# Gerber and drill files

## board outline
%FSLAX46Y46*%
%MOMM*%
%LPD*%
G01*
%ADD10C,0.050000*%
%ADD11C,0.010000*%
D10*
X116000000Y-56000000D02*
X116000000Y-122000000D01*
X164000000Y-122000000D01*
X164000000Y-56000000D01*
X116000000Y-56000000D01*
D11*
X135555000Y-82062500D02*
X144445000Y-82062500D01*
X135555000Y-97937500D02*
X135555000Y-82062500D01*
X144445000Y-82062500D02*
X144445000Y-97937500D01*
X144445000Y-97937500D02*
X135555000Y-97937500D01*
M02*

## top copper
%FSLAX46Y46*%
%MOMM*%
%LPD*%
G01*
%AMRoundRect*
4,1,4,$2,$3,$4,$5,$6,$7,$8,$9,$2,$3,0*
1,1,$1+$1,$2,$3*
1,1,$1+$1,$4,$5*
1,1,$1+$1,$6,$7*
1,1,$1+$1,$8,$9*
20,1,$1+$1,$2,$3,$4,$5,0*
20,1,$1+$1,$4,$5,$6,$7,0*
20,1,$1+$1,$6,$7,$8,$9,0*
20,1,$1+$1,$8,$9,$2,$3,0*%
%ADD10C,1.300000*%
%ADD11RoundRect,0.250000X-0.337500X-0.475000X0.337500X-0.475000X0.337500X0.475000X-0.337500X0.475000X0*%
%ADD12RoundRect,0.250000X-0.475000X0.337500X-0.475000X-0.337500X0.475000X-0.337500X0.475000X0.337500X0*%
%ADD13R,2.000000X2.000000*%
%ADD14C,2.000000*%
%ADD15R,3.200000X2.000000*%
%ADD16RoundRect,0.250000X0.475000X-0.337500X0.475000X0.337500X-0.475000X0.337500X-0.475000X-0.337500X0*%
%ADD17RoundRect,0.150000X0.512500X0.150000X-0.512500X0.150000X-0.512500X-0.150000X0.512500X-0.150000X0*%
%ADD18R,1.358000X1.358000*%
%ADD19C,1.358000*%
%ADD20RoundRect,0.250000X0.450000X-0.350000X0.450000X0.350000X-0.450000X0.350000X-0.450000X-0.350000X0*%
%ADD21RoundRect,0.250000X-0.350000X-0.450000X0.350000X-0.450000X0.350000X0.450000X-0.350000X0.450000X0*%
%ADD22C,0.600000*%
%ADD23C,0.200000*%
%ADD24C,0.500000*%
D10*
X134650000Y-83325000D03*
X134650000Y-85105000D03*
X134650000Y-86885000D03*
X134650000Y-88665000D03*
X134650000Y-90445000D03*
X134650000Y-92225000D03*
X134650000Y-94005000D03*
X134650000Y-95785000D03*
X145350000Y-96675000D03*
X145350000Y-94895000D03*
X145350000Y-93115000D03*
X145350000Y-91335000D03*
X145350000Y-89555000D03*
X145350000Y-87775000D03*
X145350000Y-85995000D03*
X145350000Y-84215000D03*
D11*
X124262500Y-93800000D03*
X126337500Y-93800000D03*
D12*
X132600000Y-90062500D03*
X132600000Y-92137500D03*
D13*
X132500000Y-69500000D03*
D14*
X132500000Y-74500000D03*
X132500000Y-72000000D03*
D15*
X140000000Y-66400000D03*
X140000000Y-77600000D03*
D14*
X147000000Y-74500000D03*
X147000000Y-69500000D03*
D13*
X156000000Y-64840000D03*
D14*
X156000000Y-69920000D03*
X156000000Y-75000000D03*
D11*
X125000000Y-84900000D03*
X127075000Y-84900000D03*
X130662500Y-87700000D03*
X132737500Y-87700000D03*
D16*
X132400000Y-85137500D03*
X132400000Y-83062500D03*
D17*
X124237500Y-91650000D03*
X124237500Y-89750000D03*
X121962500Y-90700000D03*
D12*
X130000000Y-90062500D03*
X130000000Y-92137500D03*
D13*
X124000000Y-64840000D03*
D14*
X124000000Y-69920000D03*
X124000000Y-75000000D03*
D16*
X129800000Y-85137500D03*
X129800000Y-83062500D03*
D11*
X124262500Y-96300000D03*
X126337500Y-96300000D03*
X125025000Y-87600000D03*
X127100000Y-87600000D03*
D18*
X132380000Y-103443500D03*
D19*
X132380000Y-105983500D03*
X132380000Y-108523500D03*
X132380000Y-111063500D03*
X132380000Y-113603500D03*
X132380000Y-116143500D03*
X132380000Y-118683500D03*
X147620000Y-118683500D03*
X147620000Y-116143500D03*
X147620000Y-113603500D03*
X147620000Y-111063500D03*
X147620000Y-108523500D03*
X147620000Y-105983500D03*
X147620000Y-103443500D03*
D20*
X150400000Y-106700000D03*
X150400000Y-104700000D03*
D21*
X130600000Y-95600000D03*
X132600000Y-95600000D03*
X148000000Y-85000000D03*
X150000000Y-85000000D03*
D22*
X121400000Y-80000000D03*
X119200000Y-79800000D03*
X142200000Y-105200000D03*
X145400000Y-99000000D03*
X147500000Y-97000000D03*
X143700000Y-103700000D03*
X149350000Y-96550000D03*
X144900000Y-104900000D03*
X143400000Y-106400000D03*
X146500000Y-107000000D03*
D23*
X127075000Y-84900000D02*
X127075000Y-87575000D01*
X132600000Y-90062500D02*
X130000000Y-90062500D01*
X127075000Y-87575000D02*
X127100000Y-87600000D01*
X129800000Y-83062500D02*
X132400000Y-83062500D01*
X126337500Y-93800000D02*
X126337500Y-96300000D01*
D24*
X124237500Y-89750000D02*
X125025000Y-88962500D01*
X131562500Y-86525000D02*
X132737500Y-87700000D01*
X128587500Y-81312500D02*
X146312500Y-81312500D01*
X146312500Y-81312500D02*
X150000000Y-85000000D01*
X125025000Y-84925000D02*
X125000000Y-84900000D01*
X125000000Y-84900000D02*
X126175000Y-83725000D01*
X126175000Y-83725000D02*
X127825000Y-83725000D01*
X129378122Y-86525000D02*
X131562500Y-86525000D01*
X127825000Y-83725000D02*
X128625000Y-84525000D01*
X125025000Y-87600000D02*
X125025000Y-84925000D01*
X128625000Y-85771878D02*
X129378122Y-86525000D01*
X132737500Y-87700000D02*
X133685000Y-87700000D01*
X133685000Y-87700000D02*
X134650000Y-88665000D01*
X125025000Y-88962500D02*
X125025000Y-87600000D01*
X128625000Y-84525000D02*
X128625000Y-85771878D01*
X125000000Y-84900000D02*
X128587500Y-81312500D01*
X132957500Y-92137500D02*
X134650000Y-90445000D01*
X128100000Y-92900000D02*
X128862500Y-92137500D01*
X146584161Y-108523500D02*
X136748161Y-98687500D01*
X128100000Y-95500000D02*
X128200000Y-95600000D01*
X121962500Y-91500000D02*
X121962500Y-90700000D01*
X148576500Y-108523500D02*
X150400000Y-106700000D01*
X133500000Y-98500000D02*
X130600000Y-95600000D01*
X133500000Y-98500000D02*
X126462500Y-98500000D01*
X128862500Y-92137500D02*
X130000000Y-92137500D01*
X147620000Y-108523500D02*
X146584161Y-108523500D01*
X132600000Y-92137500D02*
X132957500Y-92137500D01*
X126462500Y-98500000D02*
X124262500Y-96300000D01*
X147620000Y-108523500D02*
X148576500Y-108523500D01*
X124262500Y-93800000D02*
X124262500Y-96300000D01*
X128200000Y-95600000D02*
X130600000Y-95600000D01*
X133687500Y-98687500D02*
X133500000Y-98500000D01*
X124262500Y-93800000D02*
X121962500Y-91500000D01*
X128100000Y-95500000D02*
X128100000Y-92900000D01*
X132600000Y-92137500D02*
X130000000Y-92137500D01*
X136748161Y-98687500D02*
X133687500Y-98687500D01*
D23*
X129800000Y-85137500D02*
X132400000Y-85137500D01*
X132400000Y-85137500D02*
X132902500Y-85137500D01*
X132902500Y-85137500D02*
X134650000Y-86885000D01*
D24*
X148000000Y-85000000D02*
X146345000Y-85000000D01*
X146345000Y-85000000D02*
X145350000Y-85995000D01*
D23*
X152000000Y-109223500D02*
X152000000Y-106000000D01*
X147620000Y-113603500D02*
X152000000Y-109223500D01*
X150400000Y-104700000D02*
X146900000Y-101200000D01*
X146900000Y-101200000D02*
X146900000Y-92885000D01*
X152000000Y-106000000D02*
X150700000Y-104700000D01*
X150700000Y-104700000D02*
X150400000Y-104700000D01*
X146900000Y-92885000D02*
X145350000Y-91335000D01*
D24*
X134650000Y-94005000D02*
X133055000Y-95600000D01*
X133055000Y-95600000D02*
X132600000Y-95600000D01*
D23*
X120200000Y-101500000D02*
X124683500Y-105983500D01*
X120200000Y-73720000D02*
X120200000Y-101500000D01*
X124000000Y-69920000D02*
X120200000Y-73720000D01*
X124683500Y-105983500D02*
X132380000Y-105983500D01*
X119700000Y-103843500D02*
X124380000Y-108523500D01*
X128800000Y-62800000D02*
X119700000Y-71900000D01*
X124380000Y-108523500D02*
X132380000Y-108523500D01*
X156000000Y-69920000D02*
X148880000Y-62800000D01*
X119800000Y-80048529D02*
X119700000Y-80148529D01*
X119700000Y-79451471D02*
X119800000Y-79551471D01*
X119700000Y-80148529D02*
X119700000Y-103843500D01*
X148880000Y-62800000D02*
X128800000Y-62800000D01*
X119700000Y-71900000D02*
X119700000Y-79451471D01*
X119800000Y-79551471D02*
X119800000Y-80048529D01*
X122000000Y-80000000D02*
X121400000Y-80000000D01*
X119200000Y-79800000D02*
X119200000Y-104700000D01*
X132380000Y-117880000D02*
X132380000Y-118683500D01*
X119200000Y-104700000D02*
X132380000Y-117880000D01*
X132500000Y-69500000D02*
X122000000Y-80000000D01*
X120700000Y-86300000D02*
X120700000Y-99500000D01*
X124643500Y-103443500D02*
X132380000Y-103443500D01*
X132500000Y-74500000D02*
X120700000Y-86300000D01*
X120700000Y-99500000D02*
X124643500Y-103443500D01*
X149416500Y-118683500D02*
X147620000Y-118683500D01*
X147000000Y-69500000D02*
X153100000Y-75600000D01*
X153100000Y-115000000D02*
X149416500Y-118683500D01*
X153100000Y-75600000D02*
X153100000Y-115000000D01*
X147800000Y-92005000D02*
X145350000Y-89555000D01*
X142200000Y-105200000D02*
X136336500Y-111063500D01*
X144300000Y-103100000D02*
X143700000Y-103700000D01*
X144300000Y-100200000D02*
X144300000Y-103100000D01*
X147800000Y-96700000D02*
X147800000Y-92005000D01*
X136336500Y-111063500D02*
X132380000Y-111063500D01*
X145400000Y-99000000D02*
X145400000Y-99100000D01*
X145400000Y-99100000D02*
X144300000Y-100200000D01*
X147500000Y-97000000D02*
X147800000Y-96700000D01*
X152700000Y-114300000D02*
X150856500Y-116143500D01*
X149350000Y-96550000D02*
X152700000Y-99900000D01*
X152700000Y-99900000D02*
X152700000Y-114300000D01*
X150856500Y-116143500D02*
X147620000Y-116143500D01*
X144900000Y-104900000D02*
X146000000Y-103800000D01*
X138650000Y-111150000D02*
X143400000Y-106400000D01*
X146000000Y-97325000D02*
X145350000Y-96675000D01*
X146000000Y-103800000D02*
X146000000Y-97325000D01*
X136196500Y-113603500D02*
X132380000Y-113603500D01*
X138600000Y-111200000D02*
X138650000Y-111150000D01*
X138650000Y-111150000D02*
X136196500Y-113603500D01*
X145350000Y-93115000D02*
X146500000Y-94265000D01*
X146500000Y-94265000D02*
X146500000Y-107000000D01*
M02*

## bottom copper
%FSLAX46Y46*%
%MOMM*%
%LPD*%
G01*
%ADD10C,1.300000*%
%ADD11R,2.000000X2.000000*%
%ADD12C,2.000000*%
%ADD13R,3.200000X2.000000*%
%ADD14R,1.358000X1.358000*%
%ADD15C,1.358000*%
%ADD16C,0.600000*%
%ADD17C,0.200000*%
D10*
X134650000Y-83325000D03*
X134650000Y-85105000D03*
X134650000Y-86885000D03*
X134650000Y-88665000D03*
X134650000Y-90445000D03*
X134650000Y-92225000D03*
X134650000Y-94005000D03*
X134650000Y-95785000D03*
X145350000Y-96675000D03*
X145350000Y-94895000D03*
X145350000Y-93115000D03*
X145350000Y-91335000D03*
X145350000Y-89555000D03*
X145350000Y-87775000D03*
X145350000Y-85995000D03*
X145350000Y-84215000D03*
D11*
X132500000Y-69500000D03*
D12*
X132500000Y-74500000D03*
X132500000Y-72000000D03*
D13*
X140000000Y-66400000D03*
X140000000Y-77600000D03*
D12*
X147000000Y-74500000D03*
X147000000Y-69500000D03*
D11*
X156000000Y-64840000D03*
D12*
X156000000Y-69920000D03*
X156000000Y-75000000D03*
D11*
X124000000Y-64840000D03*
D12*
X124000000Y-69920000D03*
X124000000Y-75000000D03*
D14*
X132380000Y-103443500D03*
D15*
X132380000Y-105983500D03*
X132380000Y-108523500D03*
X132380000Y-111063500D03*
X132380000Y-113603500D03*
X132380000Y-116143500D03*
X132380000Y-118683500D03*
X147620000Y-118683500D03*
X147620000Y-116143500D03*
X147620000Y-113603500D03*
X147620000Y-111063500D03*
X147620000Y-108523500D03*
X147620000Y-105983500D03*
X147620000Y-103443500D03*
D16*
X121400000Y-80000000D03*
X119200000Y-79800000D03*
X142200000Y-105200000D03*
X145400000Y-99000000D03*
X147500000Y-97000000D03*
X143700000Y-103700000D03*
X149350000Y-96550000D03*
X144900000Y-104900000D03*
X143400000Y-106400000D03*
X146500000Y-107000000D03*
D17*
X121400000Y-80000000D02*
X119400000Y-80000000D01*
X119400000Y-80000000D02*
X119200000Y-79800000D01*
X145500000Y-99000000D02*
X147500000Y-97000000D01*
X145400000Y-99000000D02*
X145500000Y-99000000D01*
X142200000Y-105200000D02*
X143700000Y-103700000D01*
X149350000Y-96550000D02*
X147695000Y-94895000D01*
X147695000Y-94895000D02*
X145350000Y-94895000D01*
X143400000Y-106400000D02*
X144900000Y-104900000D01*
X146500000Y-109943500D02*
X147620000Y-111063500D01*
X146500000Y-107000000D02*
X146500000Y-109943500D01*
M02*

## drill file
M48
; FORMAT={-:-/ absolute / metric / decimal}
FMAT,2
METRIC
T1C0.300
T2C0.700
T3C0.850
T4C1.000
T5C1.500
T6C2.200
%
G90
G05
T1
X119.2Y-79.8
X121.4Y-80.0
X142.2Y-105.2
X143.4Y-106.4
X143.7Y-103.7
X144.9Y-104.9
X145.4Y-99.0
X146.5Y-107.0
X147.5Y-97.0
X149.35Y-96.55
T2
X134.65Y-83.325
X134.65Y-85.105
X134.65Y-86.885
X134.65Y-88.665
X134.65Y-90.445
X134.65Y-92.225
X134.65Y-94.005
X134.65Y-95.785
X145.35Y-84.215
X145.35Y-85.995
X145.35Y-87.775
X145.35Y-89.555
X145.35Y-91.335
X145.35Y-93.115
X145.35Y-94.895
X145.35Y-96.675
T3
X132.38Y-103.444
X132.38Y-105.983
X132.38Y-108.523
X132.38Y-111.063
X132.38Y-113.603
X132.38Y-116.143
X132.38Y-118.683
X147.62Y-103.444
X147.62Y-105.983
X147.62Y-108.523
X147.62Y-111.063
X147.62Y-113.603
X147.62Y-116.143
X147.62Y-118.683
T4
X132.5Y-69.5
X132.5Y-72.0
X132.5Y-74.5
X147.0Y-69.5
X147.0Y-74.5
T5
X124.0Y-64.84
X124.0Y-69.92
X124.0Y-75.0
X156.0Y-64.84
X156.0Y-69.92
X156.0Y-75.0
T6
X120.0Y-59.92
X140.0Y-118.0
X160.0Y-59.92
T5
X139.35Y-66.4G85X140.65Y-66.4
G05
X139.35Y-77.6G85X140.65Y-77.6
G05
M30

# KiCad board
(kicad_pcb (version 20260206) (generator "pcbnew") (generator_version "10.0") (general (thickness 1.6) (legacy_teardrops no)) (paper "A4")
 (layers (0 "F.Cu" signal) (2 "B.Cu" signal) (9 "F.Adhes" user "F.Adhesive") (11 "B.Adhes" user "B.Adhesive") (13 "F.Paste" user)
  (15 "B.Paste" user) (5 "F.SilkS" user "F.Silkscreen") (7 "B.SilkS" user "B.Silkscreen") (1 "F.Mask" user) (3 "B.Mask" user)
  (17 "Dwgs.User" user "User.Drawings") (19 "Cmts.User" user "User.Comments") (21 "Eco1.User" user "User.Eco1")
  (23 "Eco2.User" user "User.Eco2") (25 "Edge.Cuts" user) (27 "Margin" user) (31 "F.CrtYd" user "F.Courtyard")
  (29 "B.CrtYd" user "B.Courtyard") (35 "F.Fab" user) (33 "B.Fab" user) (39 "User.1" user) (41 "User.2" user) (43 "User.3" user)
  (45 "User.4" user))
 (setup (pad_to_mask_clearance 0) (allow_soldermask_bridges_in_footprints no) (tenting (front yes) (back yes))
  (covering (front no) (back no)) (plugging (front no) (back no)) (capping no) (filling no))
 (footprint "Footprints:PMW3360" (layer "F.Cu") (at 140 90)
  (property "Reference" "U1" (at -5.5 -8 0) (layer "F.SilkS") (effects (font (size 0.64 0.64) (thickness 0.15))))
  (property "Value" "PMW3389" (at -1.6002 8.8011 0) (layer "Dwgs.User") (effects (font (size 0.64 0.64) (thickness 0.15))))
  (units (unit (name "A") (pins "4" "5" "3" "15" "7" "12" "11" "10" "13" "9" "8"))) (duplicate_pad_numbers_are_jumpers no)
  (fp_line (start -4.445 -7.9375) (end 4.445 -7.9375) (stroke (width 0.01) (type solid)) (layer "Edge.Cuts"))
  (fp_line (start -4.445 7.9375) (end -4.445 -7.9375) (stroke (width 0.01) (type solid)) (layer "Edge.Cuts"))
  (fp_line (start 4.445 -7.9375) (end 4.445 7.9375) (stroke (width 0.01) (type solid)) (layer "Edge.Cuts"))
  (fp_line (start 4.445 7.9375) (end -4.445 7.9375) (stroke (width 0.01) (type solid)) (layer "Edge.Cuts"))
  (pad "1" thru_hole circle (at -5.35 -6.675) (size 1.3 1.3) (drill 0.7) (layers "*.Cu" "*.Mask") (remove_unused_layers no)
   (solder_mask_margin 0.102))
  (pad "2" thru_hole circle (at -5.35 -4.895) (size 1.3 1.3) (drill 0.7) (layers "*.Cu" "*.Mask") (remove_unused_layers no)
   (solder_mask_margin 0.102))
  (pad "3" thru_hole circle (at -5.35 -3.115) (size 1.3 1.3) (drill 0.7) (layers "*.Cu" "*.Mask") (remove_unused_layers no)
   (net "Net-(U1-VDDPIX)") (solder_mask_margin 0.102))
  (pad "4" thru_hole circle (at -5.35 -1.335) (size 1.3 1.3) (drill 0.7) (layers "*.Cu" "*.Mask") (remove_unused_layers no) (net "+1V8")
   (solder_mask_margin 0.102))
  (pad "5" thru_hole circle (at -5.35 0.445) (size 1.3 1.3) (drill 0.7) (layers "*.Cu" "*.Mask") (remove_unused_layers no) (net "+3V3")
   (solder_mask_margin 0.102))
  (pad "6" thru_hole circle (at -5.35 2.225) (size 1.3 1.3) (drill 0.7) (layers "*.Cu" "*.Mask") (remove_unused_layers no)
   (solder_mask_margin 0.102))
  (pad "7" thru_hole circle (at -5.35 4.005) (size 1.3 1.3) (drill 0.7) (layers "*.Cu" "*.Mask") (remove_unused_layers no)
   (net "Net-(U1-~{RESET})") (solder_mask_margin 0.102))
  (pad "8" thru_hole circle (at -5.35 5.785) (size 1.3 1.3) (drill 0.7) (layers "*.Cu" "*.Mask") (remove_unused_layers no) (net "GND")
   (solder_mask_margin 0.102))
  (pad "9" thru_hole circle (at 5.35 6.675) (size 1.3 1.3) (drill 0.7) (layers "*.Cu" "*.Mask") (remove_unused_layers no) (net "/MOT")
   (solder_mask_margin 0.102))
  (pad "10" thru_hole circle (at 5.35 4.895) (size 1.3 1.3) (drill 0.7) (layers "*.Cu" "*.Mask") (remove_unused_layers no) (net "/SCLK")
   (solder_mask_margin 0.102))
  (pad "11" thru_hole circle (at 5.35 3.115) (size 1.3 1.3) (drill 0.7) (layers "*.Cu" "*.Mask") (remove_unused_layers no) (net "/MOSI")
   (solder_mask_margin 0.102))
  (pad "12" thru_hole circle (at 5.35 1.335) (size 1.3 1.3) (drill 0.7) (layers "*.Cu" "*.Mask") (remove_unused_layers no) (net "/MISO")
   (solder_mask_margin 0.102))
  (pad "13" thru_hole circle (at 5.35 -0.445) (size 1.3 1.3) (drill 0.7) (layers "*.Cu" "*.Mask") (remove_unused_layers no) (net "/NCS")
   (solder_mask_margin 0.102))
  (pad "14" thru_hole circle (at 5.35 -2.225) (size 1.3 1.3) (drill 0.7) (layers "*.Cu" "*.Mask") (remove_unused_layers no)
   (solder_mask_margin 0.102))
  (pad "15" thru_hole circle (at 5.35 -4.005) (size 1.3 1.3) (drill 0.7) (layers "*.Cu" "*.Mask") (remove_unused_layers no)
   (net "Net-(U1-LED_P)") (solder_mask_margin 0.102))
  (pad "16" thru_hole circle (at 5.35 -5.785) (size 1.3 1.3) (drill 0.7) (layers "*.Cu" "*.Mask") (remove_unused_layers no)
   (solder_mask_margin 0.102))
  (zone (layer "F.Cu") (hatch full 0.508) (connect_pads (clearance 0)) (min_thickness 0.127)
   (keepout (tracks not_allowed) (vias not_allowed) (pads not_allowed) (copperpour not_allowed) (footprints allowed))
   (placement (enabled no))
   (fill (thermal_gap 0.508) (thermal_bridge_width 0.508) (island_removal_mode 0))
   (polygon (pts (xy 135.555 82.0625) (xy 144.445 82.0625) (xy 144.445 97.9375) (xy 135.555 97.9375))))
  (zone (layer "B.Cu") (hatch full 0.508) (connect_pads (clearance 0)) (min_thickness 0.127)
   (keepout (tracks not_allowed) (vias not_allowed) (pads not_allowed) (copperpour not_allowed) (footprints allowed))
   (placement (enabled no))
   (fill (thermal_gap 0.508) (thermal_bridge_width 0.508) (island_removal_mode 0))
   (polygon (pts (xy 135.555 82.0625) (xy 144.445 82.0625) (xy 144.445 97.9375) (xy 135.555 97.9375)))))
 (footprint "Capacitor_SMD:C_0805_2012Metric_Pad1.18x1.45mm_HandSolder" (layer "F.Cu") (at 125.3 93.8)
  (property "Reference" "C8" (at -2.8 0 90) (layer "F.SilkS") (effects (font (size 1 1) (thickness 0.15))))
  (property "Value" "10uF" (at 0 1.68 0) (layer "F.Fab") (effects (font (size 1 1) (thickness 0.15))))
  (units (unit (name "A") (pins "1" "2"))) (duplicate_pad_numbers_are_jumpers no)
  (pad "1" smd roundrect (at -1.0375 0) (size 1.175 1.45) (layers "F.Cu" "F.Mask" "F.Paste") (roundrect_rratio 0.212766) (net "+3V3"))
  (pad "2" smd roundrect (at 1.0375 0) (size 1.175 1.45) (layers "F.Cu" "F.Mask" "F.Paste") (roundrect_rratio 0.212766) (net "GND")))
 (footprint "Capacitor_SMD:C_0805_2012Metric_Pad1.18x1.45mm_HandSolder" (layer "F.Cu") (at 132.6 91.1 -90)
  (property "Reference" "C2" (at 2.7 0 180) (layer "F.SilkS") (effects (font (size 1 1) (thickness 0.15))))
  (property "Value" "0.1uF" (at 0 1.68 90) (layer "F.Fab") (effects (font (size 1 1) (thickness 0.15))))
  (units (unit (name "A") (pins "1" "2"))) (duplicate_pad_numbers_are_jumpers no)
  (pad "1" smd roundrect (at -1.0375 0 270) (size 1.175 1.45) (layers "F.Cu" "F.Mask" "F.Paste") (roundrect_rratio 0.212766) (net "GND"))
  (pad "2" smd roundrect (at 1.0375 0 270) (size 1.175 1.45) (layers "F.Cu" "F.Mask" "F.Paste") (roundrect_rratio 0.212766) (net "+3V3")))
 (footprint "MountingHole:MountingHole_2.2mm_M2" (layer "F.Cu") (at 140 118)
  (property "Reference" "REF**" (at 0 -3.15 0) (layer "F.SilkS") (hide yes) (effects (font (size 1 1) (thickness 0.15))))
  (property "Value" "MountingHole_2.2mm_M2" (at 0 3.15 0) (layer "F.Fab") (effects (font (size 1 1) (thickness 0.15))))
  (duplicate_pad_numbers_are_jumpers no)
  (pad "" np_thru_hole circle (at 0 0) (size 2.2 2.2) (drill 2.2) (layers "*.Cu" "*.Mask")))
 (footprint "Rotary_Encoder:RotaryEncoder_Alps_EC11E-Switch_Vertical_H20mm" (layer "F.Cu") (at 132.5 69.5)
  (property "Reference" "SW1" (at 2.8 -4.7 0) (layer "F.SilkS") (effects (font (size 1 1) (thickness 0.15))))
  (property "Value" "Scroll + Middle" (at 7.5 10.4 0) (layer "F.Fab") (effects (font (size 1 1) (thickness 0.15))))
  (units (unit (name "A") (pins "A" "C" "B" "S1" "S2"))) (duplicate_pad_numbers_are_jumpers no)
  (pad "A" thru_hole rect (at 0 0) (size 2 2) (drill 1) (layers "*.Cu" "*.Mask") (remove_unused_layers no) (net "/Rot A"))
  (pad "B" thru_hole circle (at 0 5) (size 2 2) (drill 1) (layers "*.Cu" "*.Mask") (remove_unused_layers no) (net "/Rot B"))
  (pad "C" thru_hole circle (at 0 2.5) (size 2 2) (drill 1) (layers "*.Cu" "*.Mask") (remove_unused_layers no) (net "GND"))
  (pad "MP" thru_hole rect (at 7.5 -3.1) (size 3.2 2) (drill oval 2.8 1.5) (layers "*.Cu" "*.Mask") (remove_unused_layers no))
  (pad "MP" thru_hole rect (at 7.5 8.1) (size 3.2 2) (drill oval 2.8 1.5) (layers "*.Cu" "*.Mask") (remove_unused_layers no))
  (pad "S1" thru_hole circle (at 14.5 5) (size 2 2) (drill 1) (layers "*.Cu" "*.Mask") (remove_unused_layers no) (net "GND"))
  (pad "S2" thru_hole circle (at 14.5 0) (size 2 2) (drill 1) (layers "*.Cu" "*.Mask") (remove_unused_layers no) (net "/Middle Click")))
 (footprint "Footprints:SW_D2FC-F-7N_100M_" (layer "F.Cu") (at 156 69.92 -90)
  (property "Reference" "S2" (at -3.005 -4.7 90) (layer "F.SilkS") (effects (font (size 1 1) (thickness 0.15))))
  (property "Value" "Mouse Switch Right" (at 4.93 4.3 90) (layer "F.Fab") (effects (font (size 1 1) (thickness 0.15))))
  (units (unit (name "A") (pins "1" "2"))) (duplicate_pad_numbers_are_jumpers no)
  (pad "1" thru_hole rect (at -5.08 0 270) (size 2 2) (drill 1.5) (layers "*.Cu" "*.Mask") (remove_unused_layers no) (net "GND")
   (solder_mask_margin 0.102))
  (pad "2" thru_hole circle (at 0 0 270) (size 2 2) (drill 1.5) (layers "*.Cu" "*.Mask") (remove_unused_layers no) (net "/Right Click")
   (solder_mask_margin 0.102))
  (pad "3" thru_hole circle (at 5.08 0 270) (size 2 2) (drill 1.5) (layers "*.Cu" "*.Mask") (remove_unused_layers no)
   (solder_mask_margin 0.102)))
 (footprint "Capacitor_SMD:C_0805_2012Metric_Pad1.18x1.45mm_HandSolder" (layer "F.Cu") (at 126.0375 84.9)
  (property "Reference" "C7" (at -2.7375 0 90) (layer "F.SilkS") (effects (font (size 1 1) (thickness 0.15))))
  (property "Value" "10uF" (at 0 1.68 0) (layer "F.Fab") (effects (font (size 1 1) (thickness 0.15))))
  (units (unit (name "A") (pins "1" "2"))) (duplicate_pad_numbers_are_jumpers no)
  (pad "1" smd roundrect (at -1.0375 0) (size 1.175 1.45) (layers "F.Cu" "F.Mask" "F.Paste") (roundrect_rratio 0.212766) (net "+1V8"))
  (pad "2" smd roundrect (at 1.0375 0) (size 1.175 1.45) (layers "F.Cu" "F.Mask" "F.Paste") (roundrect_rratio 0.212766) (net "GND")))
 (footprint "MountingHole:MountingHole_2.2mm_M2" (layer "F.Cu") (at 120 59.92)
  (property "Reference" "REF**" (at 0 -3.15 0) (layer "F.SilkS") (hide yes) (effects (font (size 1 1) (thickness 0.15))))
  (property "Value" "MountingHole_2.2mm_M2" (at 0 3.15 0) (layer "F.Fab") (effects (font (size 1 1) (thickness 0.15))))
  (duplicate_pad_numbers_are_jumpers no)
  (pad "" np_thru_hole circle (at 0 0) (size 2.2 2.2) (drill 2.2) (layers "*.Cu" "*.Mask")))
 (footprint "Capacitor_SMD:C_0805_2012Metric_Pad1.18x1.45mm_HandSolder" (layer "F.Cu") (at 131.7 87.7)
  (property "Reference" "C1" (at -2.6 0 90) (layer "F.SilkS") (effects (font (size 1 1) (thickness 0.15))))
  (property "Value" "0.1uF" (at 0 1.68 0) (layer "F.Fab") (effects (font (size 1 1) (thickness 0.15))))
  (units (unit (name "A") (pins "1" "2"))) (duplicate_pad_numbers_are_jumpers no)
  (pad "1" smd roundrect (at -1.0375 0) (size 1.175 1.45) (layers "F.Cu" "F.Mask" "F.Paste") (roundrect_rratio 0.212766) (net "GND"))
  (pad "2" smd roundrect (at 1.0375 0) (size 1.175 1.45) (layers "F.Cu" "F.Mask" "F.Paste") (roundrect_rratio 0.212766) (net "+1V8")))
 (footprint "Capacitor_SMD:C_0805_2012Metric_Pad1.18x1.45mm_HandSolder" (layer "F.Cu") (at 132.4 84.1 90)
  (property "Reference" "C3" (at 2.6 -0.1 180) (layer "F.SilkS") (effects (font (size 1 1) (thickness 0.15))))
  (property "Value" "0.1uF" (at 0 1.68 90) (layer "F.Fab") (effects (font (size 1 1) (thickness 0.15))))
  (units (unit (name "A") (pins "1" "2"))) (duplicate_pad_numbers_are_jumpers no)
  (pad "1" smd roundrect (at -1.0375 0 90) (size 1.175 1.45) (layers "F.Cu" "F.Mask" "F.Paste") (roundrect_rratio 0.212766)
   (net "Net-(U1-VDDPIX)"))
  (pad "2" smd roundrect (at 1.0375 0 90) (size 1.175 1.45) (layers "F.Cu" "F.Mask" "F.Paste") (roundrect_rratio 0.212766) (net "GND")))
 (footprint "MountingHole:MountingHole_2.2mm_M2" (layer "F.Cu") (at 160 59.92)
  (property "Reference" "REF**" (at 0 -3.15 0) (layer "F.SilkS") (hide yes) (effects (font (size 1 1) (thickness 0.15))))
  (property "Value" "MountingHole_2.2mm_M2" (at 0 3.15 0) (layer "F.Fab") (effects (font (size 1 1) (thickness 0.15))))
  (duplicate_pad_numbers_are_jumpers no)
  (pad "" np_thru_hole circle (at 0 0) (size 2.2 2.2) (drill 2.2) (layers "*.Cu" "*.Mask")))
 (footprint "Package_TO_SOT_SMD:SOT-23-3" (layer "F.Cu") (at 123.1 90.7 180)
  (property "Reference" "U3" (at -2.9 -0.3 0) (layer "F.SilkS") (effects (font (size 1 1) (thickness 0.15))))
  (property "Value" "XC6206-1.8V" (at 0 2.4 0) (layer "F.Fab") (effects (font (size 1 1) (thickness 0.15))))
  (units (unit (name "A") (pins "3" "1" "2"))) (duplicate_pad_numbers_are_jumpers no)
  (pad "1" smd roundrect (at -1.1375 -0.95 180) (size 1.325 0.6) (layers "F.Cu" "F.Mask" "F.Paste") (roundrect_rratio 0.25) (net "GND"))
  (pad "2" smd roundrect (at -1.1375 0.95 180) (size 1.325 0.6) (layers "F.Cu" "F.Mask" "F.Paste") (roundrect_rratio 0.25) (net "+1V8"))
  (pad "3" smd roundrect (at 1.1375 0 180) (size 1.325 0.6) (layers "F.Cu" "F.Mask" "F.Paste") (roundrect_rratio 0.25) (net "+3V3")))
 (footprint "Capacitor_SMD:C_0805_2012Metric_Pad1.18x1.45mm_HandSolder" (layer "F.Cu") (at 130 91.1 -90)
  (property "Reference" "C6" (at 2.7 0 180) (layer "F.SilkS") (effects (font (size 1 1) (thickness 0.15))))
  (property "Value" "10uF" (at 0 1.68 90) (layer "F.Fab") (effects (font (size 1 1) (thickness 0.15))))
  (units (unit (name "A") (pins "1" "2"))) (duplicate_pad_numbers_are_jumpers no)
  (pad "1" smd roundrect (at -1.0375 0 270) (size 1.175 1.45) (layers "F.Cu" "F.Mask" "F.Paste") (roundrect_rratio 0.212766) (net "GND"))
  (pad "2" smd roundrect (at 1.0375 0 270) (size 1.175 1.45) (layers "F.Cu" "F.Mask" "F.Paste") (roundrect_rratio 0.212766) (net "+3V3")))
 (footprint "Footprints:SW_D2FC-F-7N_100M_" (layer "F.Cu") (at 124 69.92 -90)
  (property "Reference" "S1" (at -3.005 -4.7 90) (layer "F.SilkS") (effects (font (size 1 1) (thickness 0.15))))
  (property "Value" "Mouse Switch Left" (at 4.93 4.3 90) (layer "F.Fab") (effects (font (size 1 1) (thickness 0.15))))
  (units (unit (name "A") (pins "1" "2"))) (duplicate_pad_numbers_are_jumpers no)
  (pad "1" thru_hole rect (at -5.08 0 270) (size 2 2) (drill 1.5) (layers "*.Cu" "*.Mask") (remove_unused_layers no) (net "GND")
   (solder_mask_margin 0.102))
  (pad "2" thru_hole circle (at 0 0 270) (size 2 2) (drill 1.5) (layers "*.Cu" "*.Mask") (remove_unused_layers no) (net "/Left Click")
   (solder_mask_margin 0.102))
  (pad "3" thru_hole circle (at 5.08 0 270) (size 2 2) (drill 1.5) (layers "*.Cu" "*.Mask") (remove_unused_layers no)
   (solder_mask_margin 0.102)))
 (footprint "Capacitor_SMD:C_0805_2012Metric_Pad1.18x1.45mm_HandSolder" (layer "F.Cu") (at 129.8 84.1 90)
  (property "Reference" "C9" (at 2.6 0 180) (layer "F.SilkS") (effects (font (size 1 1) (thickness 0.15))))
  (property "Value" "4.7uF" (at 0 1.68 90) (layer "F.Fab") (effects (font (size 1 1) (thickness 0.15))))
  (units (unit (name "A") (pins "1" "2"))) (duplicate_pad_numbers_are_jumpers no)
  (pad "1" smd roundrect (at -1.0375 0 90) (size 1.175 1.45) (layers "F.Cu" "F.Mask" "F.Paste") (roundrect_rratio 0.212766)
   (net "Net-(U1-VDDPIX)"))
  (pad "2" smd roundrect (at 1.0375 0 90) (size 1.175 1.45) (layers "F.Cu" "F.Mask" "F.Paste") (roundrect_rratio 0.212766) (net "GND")))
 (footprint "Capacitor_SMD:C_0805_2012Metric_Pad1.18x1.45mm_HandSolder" (layer "F.Cu") (at 125.3 96.3)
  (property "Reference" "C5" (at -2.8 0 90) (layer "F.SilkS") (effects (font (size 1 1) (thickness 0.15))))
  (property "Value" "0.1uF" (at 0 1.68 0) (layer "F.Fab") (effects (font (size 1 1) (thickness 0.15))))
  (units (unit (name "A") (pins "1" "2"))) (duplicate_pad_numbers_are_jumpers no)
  (pad "1" smd roundrect (at -1.0375 0) (size 1.175 1.45) (layers "F.Cu" "F.Mask" "F.Paste") (roundrect_rratio 0.212766) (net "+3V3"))
  (pad "2" smd roundrect (at 1.0375 0) (size 1.175 1.45) (layers "F.Cu" "F.Mask" "F.Paste") (roundrect_rratio 0.212766) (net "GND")))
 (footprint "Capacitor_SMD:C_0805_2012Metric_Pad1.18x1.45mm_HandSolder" (layer "F.Cu") (at 126.0625 87.6)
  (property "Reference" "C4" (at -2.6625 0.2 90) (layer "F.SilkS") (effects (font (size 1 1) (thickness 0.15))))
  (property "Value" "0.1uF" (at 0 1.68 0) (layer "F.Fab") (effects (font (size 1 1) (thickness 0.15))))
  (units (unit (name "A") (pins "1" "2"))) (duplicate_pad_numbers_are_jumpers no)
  (pad "1" smd roundrect (at -1.0375 0) (size 1.175 1.45) (layers "F.Cu" "F.Mask" "F.Paste") (roundrect_rratio 0.212766) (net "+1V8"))
  (pad "2" smd roundrect (at 1.0375 0) (size 1.175 1.45) (layers "F.Cu" "F.Mask" "F.Paste") (roundrect_rratio 0.212766) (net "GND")))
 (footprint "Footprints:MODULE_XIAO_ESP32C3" (layer "F.Cu") (at 140 111)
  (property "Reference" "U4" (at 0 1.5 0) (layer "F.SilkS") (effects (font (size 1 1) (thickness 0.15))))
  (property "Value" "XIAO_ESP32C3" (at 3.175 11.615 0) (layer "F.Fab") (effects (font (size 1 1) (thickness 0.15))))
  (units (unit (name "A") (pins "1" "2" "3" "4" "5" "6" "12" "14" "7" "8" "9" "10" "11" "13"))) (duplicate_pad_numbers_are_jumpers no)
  (pad "1" thru_hole rect (at -7.62 -7.5565) (size 1.358 1.358) (drill 0.85) (layers "*.Cu" "*.Mask") (remove_unused_layers no)
   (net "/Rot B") (solder_mask_margin 0.102))
  (pad "2" thru_hole circle (at -7.62 -5.0165) (size 1.358 1.358) (drill 0.85) (layers "*.Cu" "*.Mask") (remove_unused_layers no)
   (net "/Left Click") (solder_mask_margin 0.102))
  (pad "3" thru_hole circle (at -7.62 -2.4765) (size 1.358 1.358) (drill 0.85) (layers "*.Cu" "*.Mask") (remove_unused_layers no)
   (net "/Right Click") (solder_mask_margin 0.102))
  (pad "4" thru_hole circle (at -7.62 0.0635) (size 1.358 1.358) (drill 0.85) (layers "*.Cu" "*.Mask") (remove_unused_layers no)
   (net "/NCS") (solder_mask_margin 0.102))
  (pad "5" thru_hole circle (at -7.62 2.6035) (size 1.358 1.358) (drill 0.85) (layers "*.Cu" "*.Mask") (remove_unused_layers no)
   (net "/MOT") (solder_mask_margin 0.102))
  (pad "6" thru_hole circle (at -7.62 5.1435) (size 1.358 1.358) (drill 0.85) (layers "*.Cu" "*.Mask") (remove_unused_layers no)
   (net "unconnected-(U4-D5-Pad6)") (solder_mask_margin 0.102))
  (pad "7" thru_hole circle (at -7.62 7.6835) (size 1.358 1.358) (drill 0.85) (layers "*.Cu" "*.Mask") (remove_unused_layers no)
   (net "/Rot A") (solder_mask_margin 0.102))
  (pad "8" thru_hole circle (at 7.62 7.6835) (size 1.358 1.358) (drill 0.85) (layers "*.Cu" "*.Mask") (remove_unused_layers no)
   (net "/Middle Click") (solder_mask_margin 0.102))
  (pad "9" thru_hole circle (at 7.62 5.1435) (size 1.358 1.358) (drill 0.85) (layers "*.Cu" "*.Mask") (remove_unused_layers no)
   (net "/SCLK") (solder_mask_margin 0.102))
  (pad "10" thru_hole circle (at 7.62 2.6035) (size 1.358 1.358) (drill 0.85) (layers "*.Cu" "*.Mask") (remove_unused_layers no)
   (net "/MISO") (solder_mask_margin 0.102))
  (pad "11" thru_hole circle (at 7.62 0.0635) (size 1.358 1.358) (drill 0.85) (layers "*.Cu" "*.Mask") (remove_unused_layers no)
   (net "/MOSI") (solder_mask_margin 0.102))
  (pad "12" thru_hole circle (at 7.62 -2.4765) (size 1.358 1.358) (drill 0.85) (layers "*.Cu" "*.Mask") (remove_unused_layers no)
   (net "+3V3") (solder_mask_margin 0.102))
  (pad "13" thru_hole circle (at 7.62 -5.0165) (size 1.358 1.358) (drill 0.85) (layers "*.Cu" "*.Mask") (remove_unused_layers no)
   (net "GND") (solder_mask_margin 0.102))
  (pad "14" thru_hole circle (at 7.62 -7.5565) (size 1.358 1.358) (drill 0.85) (layers "*.Cu" "*.Mask") (remove_unused_layers no)
   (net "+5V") (solder_mask_margin 0.102)))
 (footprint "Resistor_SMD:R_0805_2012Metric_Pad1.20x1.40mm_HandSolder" (layer "F.Cu") (at 150.4 105.7 90)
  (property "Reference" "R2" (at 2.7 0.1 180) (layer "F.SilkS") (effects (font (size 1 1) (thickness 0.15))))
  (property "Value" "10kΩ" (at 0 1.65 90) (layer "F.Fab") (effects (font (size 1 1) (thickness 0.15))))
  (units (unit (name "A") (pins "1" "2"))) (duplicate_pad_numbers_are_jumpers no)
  (pad "1" smd roundrect (at -1 0 90) (size 1.2 1.4) (layers "F.Cu" "F.Mask" "F.Paste") (roundrect_rratio 0.208333) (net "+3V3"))
  (pad "2" smd roundrect (at 1 0 90) (size 1.2 1.4) (layers "F.Cu" "F.Mask" "F.Paste") (roundrect_rratio 0.208333) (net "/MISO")))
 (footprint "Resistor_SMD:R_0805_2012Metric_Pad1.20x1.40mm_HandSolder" (layer "F.Cu") (at 131.6 95.6)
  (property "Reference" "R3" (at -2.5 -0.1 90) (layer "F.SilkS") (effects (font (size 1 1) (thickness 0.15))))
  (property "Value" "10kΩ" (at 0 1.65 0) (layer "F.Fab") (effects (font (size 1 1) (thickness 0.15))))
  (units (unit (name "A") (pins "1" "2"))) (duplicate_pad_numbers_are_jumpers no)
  (pad "1" smd roundrect (at -1 0) (size 1.2 1.4) (layers "F.Cu" "F.Mask" "F.Paste") (roundrect_rratio 0.208333) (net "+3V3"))
  (pad "2" smd roundrect (at 1 0) (size 1.2 1.4) (layers "F.Cu" "F.Mask" "F.Paste") (roundrect_rratio 0.208333) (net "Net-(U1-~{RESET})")))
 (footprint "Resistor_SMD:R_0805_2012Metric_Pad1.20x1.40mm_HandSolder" (layer "F.Cu") (at 149 85)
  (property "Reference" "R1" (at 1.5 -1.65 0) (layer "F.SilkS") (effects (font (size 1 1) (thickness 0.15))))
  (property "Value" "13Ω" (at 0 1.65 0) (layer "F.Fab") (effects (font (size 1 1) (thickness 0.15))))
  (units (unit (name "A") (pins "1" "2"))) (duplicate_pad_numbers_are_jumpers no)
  (pad "1" smd roundrect (at -1 0) (size 1.2 1.4) (layers "F.Cu" "F.Mask" "F.Paste") (roundrect_rratio 0.208333) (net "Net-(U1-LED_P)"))
  (pad "2" smd roundrect (at 1 0) (size 1.2 1.4) (layers "F.Cu" "F.Mask" "F.Paste") (roundrect_rratio 0.208333) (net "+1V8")))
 (gr_poly (pts (xy 116 56) (xy 116 122) (xy 164 122) (xy 164 56)) (stroke (width 0.05) (type solid)) (fill no) (layer "Edge.Cuts"))
 (segment (start 127.075 84.9) (end 127.075 87.575) (width 0.2) (layer "F.Cu") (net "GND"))
 (segment (start 132.6 90.0625) (end 130 90.0625) (width 0.2) (layer "F.Cu") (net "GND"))
 (segment (start 127.075 87.575) (end 127.1 87.6) (width 0.2) (layer "F.Cu") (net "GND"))
 (segment (start 129.8 83.0625) (end 132.4 83.0625) (width 0.2) (layer "F.Cu") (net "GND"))
 (segment (start 126.3375 93.8) (end 126.3375 96.3) (width 0.2) (layer "F.Cu") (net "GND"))
 (segment (start 124.2375 89.75) (end 125.025 88.9625) (width 0.5) (layer "F.Cu") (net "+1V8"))
 (segment (start 131.5625 86.525) (end 132.7375 87.7) (width 0.5) (layer "F.Cu") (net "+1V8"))
 (segment (start 128.5875 81.3125) (end 146.3125 81.3125) (width 0.5) (layer "F.Cu") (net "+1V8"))
 (segment (start 146.3125 81.3125) (end 150 85) (width 0.5) (layer "F.Cu") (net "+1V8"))
 (segment (start 125.025 84.925) (end 125 84.9) (width 0.5) (layer "F.Cu") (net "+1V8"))
 (segment (start 125 84.9) (end 126.175 83.725) (width 0.5) (layer "F.Cu") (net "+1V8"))
 (segment (start 126.175 83.725) (end 127.825 83.725) (width 0.5) (layer "F.Cu") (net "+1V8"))
 (segment (start 129.378122 86.525) (end 131.5625 86.525) (width 0.5) (layer "F.Cu") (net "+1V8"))
 (segment (start 127.825 83.725) (end 128.625 84.525) (width 0.5) (layer "F.Cu") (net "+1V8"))
 (segment (start 125.025 87.6) (end 125.025 84.925) (width 0.5) (layer "F.Cu") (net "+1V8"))
 (segment (start 128.625 85.771878) (end 129.378122 86.525) (width 0.5) (layer "F.Cu") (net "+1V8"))
 (segment (start 132.7375 87.7) (end 133.685 87.7) (width 0.5) (layer "F.Cu") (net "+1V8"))
 (segment (start 133.685 87.7) (end 134.65 88.665) (width 0.5) (layer "F.Cu") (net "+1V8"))
 (segment (start 125.025 88.9625) (end 125.025 87.6) (width 0.5) (layer "F.Cu") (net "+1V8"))
 (segment (start 128.625 84.525) (end 128.625 85.771878) (width 0.5) (layer "F.Cu") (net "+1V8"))
 (segment (start 125 84.9) (end 128.5875 81.3125) (width 0.5) (layer "F.Cu") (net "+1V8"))
 (segment (start 132.9575 92.1375) (end 134.65 90.445) (width 0.5) (layer "F.Cu") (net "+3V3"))
 (segment (start 128.1 92.9) (end 128.8625 92.1375) (width 0.5) (layer "F.Cu") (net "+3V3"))
 (segment (start 146.584161 108.5235) (end 136.748161 98.6875) (width 0.5) (layer "F.Cu") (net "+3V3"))
 (segment (start 128.1 95.5) (end 128.2 95.6) (width 0.5) (layer "F.Cu") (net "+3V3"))
 (segment (start 121.9625 91.5) (end 121.9625 90.7) (width 0.5) (layer "F.Cu") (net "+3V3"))
 (segment (start 148.5765 108.5235) (end 150.4 106.7) (width 0.5) (layer "F.Cu") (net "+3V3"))
 (segment (start 133.5 98.5) (end 130.6 95.6) (width 0.5) (layer "F.Cu") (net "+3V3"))
 (segment (start 133.5 98.5) (end 126.4625 98.5) (width 0.5) (layer "F.Cu") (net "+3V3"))
 (segment (start 128.8625 92.1375) (end 130 92.1375) (width 0.5) (layer "F.Cu") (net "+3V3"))
 (segment (start 147.62 108.5235) (end 146.584161 108.5235) (width 0.5) (layer "F.Cu") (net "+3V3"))
 (segment (start 132.6 92.1375) (end 132.9575 92.1375) (width 0.5) (layer "F.Cu") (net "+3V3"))
 (segment (start 126.4625 98.5) (end 124.2625 96.3) (width 0.5) (layer "F.Cu") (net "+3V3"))
 (segment (start 147.62 108.5235) (end 148.5765 108.5235) (width 0.5) (layer "F.Cu") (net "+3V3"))
 (segment (start 124.2625 93.8) (end 124.2625 96.3) (width 0.5) (layer "F.Cu") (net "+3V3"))
 (segment (start 128.2 95.6) (end 130.6 95.6) (width 0.5) (layer "F.Cu") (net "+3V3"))
 (segment (start 133.6875 98.6875) (end 133.5 98.5) (width 0.5) (layer "F.Cu") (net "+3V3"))
 (segment (start 124.2625 93.8) (end 121.9625 91.5) (width 0.5) (layer "F.Cu") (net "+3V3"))
 (segment (start 128.1 95.5) (end 128.1 92.9) (width 0.5) (layer "F.Cu") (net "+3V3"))
 (segment (start 132.6 92.1375) (end 130 92.1375) (width 0.5) (layer "F.Cu") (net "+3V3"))
 (segment (start 136.748161 98.6875) (end 133.6875 98.6875) (width 0.5) (layer "F.Cu") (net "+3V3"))
 (segment (start 129.8 85.1375) (end 132.4 85.1375) (width 0.2) (layer "F.Cu") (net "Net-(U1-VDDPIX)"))
 (segment (start 132.4 85.1375) (end 132.9025 85.1375) (width 0.2) (layer "F.Cu") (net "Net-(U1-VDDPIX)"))
 (segment (start 132.9025 85.1375) (end 134.65 86.885) (width 0.2) (layer "F.Cu") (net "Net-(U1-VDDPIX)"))
 (segment (start 148 85) (end 146.345 85) (width 0.5) (layer "F.Cu") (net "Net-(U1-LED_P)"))
 (segment (start 146.345 85) (end 145.35 85.995) (width 0.5) (layer "F.Cu") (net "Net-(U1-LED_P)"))
 (segment (start 152 109.2235) (end 152 106) (width 0.2) (layer "F.Cu") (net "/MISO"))
 (segment (start 147.62 113.6035) (end 152 109.2235) (width 0.2) (layer "F.Cu") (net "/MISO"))
 (segment (start 150.4 104.7) (end 146.9 101.2) (width 0.2) (layer "F.Cu") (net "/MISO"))
 (segment (start 146.9 101.2) (end 146.9 92.885) (width 0.2) (layer "F.Cu") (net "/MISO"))
 (segment (start 152 106) (end 150.7 104.7) (width 0.2) (layer "F.Cu") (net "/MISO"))
 (segment (start 150.7 104.7) (end 150.4 104.7) (width 0.2) (layer "F.Cu") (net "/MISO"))
 (segment (start 146.9 92.885) (end 145.35 91.335) (width 0.2) (layer "F.Cu") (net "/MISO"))
 (segment (start 134.65 94.005) (end 133.055 95.6) (width 0.5) (layer "F.Cu") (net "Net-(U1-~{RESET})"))
 (segment (start 133.055 95.6) (end 132.6 95.6) (width 0.5) (layer "F.Cu") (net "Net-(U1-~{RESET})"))
 (segment (start 120.2 101.5) (end 124.6835 105.9835) (width 0.2) (layer "F.Cu") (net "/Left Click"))
 (segment (start 120.2 73.72) (end 120.2 101.5) (width 0.2) (layer "F.Cu") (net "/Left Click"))
 (segment (start 124 69.92) (end 120.2 73.72) (width 0.2) (layer "F.Cu") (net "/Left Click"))
 (segment (start 124.6835 105.9835) (end 132.38 105.9835) (width 0.2) (layer "F.Cu") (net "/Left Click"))
 (segment (start 119.7 103.8435) (end 124.38 108.5235) (width 0.2) (layer "F.Cu") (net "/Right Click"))
 (segment (start 128.8 62.8) (end 119.7 71.9) (width 0.2) (layer "F.Cu") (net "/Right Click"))
 (segment (start 124.38 108.5235) (end 132.38 108.5235) (width 0.2) (layer "F.Cu") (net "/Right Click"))
 (segment (start 156 69.92) (end 148.88 62.8) (width 0.2) (layer "F.Cu") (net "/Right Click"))
 (segment (start 119.8 80.048529) (end 119.7 80.148529) (width 0.2) (layer "F.Cu") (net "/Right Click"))
 (segment (start 119.7 79.451471) (end 119.8 79.551471) (width 0.2) (layer "F.Cu") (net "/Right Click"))
 (segment (start 119.7 80.148529) (end 119.7 103.8435) (width 0.2) (layer "F.Cu") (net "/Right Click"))
 (segment (start 148.88 62.8) (end 128.8 62.8) (width 0.2) (layer "F.Cu") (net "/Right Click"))
 (segment (start 119.7 71.9) (end 119.7 79.451471) (width 0.2) (layer "F.Cu") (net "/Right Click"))
 (segment (start 119.8 79.551471) (end 119.8 80.048529) (width 0.2) (layer "F.Cu") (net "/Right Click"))
 (segment (start 122 80) (end 121.4 80) (width 0.2) (layer "F.Cu") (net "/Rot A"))
 (segment (start 119.2 79.8) (end 119.2 104.7) (width 0.2) (layer "F.Cu") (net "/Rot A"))
 (segment (start 132.38 117.88) (end 132.38 118.6835) (width 0.2) (layer "F.Cu") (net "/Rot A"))
 (segment (start 119.2 104.7) (end 132.38 117.88) (width 0.2) (layer "F.Cu") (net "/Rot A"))
 (segment (start 132.5 69.5) (end 122 80) (width 0.2) (layer "F.Cu") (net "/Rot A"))
 (via (at 121.4 80) (size 0.6) (drill 0.3) (layers "F.Cu" "B.Cu") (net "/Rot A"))
 (via (at 119.2 79.8) (size 0.6) (drill 0.3) (layers "F.Cu" "B.Cu") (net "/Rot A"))
 (segment (start 121.4 80) (end 119.4 80) (width 0.2) (layer "B.Cu") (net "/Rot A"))
 (segment (start 119.4 80) (end 119.2 79.8) (width 0.2) (layer "B.Cu") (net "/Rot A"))
 (segment (start 120.7 86.3) (end 120.7 99.5) (width 0.2) (layer "F.Cu") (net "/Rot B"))
 (segment (start 124.6435 103.4435) (end 132.38 103.4435) (width 0.2) (layer "F.Cu") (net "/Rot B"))
 (segment (start 132.5 74.5) (end 120.7 86.3) (width 0.2) (layer "F.Cu") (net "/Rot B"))
 (segment (start 120.7 99.5) (end 124.6435 103.4435) (width 0.2) (layer "F.Cu") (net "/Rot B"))
 (segment (start 149.4165 118.6835) (end 147.62 118.6835) (width 0.2) (layer "F.Cu") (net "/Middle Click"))
 (segment (start 147 69.5) (end 153.1 75.6) (width 0.2) (layer "F.Cu") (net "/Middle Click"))
 (segment (start 153.1 115) (end 149.4165 118.6835) (width 0.2) (layer "F.Cu") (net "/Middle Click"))
 (segment (start 153.1 75.6) (end 153.1 115) (width 0.2) (layer "F.Cu") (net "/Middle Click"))
 (segment (start 147.8 92.005) (end 145.35 89.555) (width 0.2) (layer "F.Cu") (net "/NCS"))
 (segment (start 142.2 105.2) (end 136.3365 111.0635) (width 0.2) (layer "F.Cu") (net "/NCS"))
 (segment (start 144.3 103.1) (end 143.7 103.7) (width 0.2) (layer "F.Cu") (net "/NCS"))
 (segment (start 144.3 100.2) (end 144.3 103.1) (width 0.2) (layer "F.Cu") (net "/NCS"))
 (segment (start 147.8 96.7) (end 147.8 92.005) (width 0.2) (layer "F.Cu") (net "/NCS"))
 (segment (start 136.3365 111.0635) (end 132.38 111.0635) (width 0.2) (layer "F.Cu") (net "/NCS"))
 (segment (start 145.4 99) (end 145.4 99.1) (width 0.2) (layer "F.Cu") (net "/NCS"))
 (segment (start 145.4 99.1) (end 144.3 100.2) (width 0.2) (layer "F.Cu") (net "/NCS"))
 (segment (start 147.5 97) (end 147.8 96.7) (width 0.2) (layer "F.Cu") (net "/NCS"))
 (via (at 142.2 105.2) (size 0.6) (drill 0.3) (layers "F.Cu" "B.Cu") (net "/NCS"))
 (via (at 145.4 99) (size 0.6) (drill 0.3) (layers "F.Cu" "B.Cu") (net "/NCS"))
 (via (at 147.5 97) (size 0.6) (drill 0.3) (layers "F.Cu" "B.Cu") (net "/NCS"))
 (via (at 143.7 103.7) (size 0.6) (drill 0.3) (layers "F.Cu" "B.Cu") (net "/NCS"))
 (segment (start 145.5 99) (end 147.5 97) (width 0.2) (layer "B.Cu") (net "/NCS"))
 (segment (start 145.4 99) (end 145.5 99) (width 0.2) (layer "B.Cu") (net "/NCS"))
 (segment (start 142.2 105.2) (end 143.7 103.7) (width 0.2) (layer "B.Cu") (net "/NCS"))
 (segment (start 152.7 114.3) (end 150.8565 116.1435) (width 0.2) (layer "F.Cu") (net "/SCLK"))
 (segment (start 149.35 96.55) (end 152.7 99.9) (width 0.2) (layer "F.Cu") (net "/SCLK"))
 (segment (start 152.7 99.9) (end 152.7 114.3) (width 0.2) (layer "F.Cu") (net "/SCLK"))
 (segment (start 150.8565 116.1435) (end 147.62 116.1435) (width 0.2) (layer "F.Cu") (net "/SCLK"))
 (via (at 149.35 96.55) (size 0.6) (drill 0.3) (layers "F.Cu" "B.Cu") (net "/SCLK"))
 (segment (start 149.35 96.55) (end 147.695 94.895) (width 0.2) (layer "B.Cu") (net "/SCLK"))
 (segment (start 147.695 94.895) (end 145.35 94.895) (width 0.2) (layer "B.Cu") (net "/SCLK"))
 (segment (start 144.9 104.9) (end 146 103.8) (width 0.2) (layer "F.Cu") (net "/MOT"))
 (segment (start 138.65 111.15) (end 143.4 106.4) (width 0.2) (layer "F.Cu") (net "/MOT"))
 (segment (start 146 97.325) (end 145.35 96.675) (width 0.2) (layer "F.Cu") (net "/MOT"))
 (segment (start 146 103.8) (end 146 97.325) (width 0.2) (layer "F.Cu") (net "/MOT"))
 (segment (start 136.1965 113.6035) (end 132.38 113.6035) (width 0.2) (layer "F.Cu") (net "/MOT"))
 (segment (start 138.6 111.2) (end 138.65 111.15) (width 0.2) (layer "F.Cu") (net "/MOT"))
 (segment (start 138.65 111.15) (end 136.1965 113.6035) (width 0.2) (layer "F.Cu") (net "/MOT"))
 (via (at 144.9 104.9) (size 0.6) (drill 0.3) (layers "F.Cu" "B.Cu") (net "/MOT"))
 (via (at 143.4 106.4) (size 0.6) (drill 0.3) (layers "F.Cu" "B.Cu") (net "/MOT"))
 (segment (start 143.4 106.4) (end 144.9 104.9) (width 0.2) (layer "B.Cu") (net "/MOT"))
 (segment (start 145.35 93.115) (end 146.5 94.265) (width 0.2) (layer "F.Cu") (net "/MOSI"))
 (segment (start 146.5 94.265) (end 146.5 107) (width 0.2) (layer "F.Cu") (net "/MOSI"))
 (via (at 146.5 107) (size 0.6) (drill 0.3) (layers "F.Cu" "B.Cu") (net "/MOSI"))
 (segment (start 146.5 109.9435) (end 147.62 111.0635) (width 0.2) (layer "B.Cu") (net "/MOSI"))
 (segment (start 146.5 107) (end 146.5 109.9435) (width 0.2) (layer "B.Cu") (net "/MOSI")))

